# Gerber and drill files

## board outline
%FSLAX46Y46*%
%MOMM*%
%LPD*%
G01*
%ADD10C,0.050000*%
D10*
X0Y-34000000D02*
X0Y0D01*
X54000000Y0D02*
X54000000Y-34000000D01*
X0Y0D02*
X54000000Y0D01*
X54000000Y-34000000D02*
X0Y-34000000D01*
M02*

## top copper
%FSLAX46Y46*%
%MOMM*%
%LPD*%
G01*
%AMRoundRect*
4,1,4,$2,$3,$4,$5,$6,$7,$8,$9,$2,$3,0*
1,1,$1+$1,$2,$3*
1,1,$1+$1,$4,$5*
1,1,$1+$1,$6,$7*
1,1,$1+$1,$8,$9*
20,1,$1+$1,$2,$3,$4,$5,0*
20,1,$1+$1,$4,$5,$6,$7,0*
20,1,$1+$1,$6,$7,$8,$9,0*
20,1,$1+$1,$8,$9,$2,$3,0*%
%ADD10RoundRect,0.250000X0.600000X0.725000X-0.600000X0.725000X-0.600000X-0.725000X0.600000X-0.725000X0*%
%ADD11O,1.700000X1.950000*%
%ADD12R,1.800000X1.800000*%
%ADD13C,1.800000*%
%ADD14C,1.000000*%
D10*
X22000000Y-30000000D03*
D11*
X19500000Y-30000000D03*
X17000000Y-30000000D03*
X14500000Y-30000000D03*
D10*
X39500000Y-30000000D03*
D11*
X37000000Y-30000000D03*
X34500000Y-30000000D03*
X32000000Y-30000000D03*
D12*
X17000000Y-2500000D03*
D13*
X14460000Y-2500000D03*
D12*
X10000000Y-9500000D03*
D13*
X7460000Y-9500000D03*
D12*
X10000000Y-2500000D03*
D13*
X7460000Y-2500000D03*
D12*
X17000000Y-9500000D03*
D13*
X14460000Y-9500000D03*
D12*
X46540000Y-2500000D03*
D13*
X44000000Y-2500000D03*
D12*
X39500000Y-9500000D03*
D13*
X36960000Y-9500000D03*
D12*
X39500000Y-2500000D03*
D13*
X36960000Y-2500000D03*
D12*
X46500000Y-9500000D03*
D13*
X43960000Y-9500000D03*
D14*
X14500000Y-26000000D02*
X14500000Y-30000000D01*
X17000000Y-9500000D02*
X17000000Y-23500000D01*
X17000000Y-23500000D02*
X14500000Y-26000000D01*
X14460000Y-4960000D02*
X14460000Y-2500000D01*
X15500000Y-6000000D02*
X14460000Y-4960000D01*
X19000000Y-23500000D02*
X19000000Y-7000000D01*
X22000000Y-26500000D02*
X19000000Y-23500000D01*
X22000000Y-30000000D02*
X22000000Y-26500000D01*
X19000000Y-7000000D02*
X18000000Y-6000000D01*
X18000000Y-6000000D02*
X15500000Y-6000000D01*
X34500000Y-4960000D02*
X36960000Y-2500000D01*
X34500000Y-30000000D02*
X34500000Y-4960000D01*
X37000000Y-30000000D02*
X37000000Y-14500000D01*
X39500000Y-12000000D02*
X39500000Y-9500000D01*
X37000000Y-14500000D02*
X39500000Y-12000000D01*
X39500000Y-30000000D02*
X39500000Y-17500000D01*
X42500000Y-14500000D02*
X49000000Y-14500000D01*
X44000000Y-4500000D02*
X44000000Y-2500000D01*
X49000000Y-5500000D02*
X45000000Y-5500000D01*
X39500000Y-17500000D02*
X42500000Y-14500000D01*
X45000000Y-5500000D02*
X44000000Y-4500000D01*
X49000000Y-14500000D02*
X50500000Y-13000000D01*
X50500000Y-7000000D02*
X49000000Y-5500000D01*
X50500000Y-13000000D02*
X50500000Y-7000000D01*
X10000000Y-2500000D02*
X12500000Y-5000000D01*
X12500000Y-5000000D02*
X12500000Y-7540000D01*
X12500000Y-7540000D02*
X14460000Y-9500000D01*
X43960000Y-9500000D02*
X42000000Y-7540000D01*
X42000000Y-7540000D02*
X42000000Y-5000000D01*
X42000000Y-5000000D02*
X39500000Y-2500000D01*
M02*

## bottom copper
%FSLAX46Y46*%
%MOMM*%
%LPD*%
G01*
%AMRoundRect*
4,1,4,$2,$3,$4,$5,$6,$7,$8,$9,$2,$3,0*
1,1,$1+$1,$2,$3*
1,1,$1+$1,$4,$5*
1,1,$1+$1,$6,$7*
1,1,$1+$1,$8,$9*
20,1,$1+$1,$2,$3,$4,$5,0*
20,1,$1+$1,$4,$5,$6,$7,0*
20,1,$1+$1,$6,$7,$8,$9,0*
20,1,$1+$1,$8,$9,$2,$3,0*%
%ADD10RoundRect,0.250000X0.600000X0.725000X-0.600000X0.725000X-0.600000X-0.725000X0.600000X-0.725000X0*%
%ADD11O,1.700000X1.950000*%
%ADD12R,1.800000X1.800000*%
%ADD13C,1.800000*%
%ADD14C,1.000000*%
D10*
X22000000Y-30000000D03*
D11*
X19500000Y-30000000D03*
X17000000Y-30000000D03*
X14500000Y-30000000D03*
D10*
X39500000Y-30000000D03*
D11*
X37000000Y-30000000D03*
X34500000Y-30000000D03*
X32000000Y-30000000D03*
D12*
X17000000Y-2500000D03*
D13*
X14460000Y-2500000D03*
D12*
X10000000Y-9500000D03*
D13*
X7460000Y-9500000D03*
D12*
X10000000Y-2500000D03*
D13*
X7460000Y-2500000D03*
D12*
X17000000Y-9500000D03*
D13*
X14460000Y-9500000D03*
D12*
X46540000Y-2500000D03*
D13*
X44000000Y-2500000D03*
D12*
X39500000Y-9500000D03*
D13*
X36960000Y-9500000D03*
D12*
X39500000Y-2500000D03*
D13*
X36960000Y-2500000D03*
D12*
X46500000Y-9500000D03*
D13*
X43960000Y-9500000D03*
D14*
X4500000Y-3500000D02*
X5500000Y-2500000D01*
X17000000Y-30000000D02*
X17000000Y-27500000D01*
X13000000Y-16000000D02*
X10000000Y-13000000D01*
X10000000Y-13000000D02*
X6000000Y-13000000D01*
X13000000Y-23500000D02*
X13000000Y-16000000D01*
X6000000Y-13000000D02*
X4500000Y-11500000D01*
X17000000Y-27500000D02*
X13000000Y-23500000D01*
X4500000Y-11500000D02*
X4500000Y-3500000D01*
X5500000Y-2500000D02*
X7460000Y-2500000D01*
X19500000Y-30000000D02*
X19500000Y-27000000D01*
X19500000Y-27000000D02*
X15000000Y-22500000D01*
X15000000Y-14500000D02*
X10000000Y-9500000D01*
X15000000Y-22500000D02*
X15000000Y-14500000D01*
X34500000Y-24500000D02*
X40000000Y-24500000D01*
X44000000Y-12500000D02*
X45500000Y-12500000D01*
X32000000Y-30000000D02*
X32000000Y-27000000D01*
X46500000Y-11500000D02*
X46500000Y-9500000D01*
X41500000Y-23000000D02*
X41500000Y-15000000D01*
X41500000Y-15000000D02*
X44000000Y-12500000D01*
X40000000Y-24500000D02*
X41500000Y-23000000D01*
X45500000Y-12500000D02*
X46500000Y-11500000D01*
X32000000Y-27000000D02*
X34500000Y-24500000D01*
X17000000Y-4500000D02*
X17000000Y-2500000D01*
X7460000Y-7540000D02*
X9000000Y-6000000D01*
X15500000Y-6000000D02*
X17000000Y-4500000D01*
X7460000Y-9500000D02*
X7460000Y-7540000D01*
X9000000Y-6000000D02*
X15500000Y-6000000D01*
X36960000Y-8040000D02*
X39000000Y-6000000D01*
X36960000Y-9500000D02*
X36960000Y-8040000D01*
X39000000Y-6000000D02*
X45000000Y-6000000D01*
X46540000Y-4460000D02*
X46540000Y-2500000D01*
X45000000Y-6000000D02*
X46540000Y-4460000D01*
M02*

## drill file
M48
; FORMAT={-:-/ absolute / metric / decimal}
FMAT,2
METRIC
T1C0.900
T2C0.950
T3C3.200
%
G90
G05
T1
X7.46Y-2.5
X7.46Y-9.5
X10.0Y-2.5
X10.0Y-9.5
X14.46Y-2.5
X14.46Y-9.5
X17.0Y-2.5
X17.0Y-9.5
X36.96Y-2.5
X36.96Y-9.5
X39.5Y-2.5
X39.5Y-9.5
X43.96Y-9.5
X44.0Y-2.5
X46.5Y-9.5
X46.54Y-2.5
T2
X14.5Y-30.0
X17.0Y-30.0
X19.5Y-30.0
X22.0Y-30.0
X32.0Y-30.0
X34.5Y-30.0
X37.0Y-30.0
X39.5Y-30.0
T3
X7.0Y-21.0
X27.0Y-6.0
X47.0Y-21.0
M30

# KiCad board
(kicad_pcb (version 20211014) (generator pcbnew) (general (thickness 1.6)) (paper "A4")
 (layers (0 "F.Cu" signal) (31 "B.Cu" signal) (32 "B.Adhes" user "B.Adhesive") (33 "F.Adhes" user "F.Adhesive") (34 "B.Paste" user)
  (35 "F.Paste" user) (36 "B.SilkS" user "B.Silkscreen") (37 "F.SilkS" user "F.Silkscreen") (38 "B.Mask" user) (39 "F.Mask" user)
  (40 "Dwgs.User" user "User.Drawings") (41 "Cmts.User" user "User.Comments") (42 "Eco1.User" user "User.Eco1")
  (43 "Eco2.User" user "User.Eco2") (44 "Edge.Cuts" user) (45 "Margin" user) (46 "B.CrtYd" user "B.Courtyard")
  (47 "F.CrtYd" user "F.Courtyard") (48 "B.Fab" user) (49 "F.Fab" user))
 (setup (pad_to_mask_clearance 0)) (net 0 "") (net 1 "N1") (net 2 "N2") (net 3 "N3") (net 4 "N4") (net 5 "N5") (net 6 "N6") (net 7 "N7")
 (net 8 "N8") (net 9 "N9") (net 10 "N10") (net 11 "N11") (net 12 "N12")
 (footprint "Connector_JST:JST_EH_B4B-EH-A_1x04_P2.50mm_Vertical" (layer "F.Cu") (at 22 30 180)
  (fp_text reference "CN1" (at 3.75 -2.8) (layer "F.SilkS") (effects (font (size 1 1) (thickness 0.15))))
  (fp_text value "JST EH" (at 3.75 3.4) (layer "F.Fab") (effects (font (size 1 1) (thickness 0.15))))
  (pad "1" thru_hole roundrect locked (at 0 0 180) (size 1.7 1.95) (drill 0.95) (layers *.Cu *.Mask) (roundrect_rratio 0.147059)
   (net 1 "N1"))
  (pad "2" thru_hole oval locked (at 2.5 0 180) (size 1.7 1.95) (drill 0.95) (layers *.Cu *.Mask) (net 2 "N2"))
  (pad "3" thru_hole oval locked (at 5 0 180) (size 1.7 1.95) (drill 0.95) (layers *.Cu *.Mask) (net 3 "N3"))
  (pad "4" thru_hole oval locked (at 7.5 0 180) (size 1.7 1.95) (drill 0.95) (layers *.Cu *.Mask) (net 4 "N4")))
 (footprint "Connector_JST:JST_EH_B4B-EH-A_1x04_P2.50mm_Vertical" (layer "F.Cu") (at 39.5 30 180)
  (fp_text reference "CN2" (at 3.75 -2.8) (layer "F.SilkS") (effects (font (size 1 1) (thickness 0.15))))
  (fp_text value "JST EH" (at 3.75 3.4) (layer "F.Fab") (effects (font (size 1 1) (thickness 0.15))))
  (pad "1" thru_hole roundrect locked (at 0 0 180) (size 1.7 1.95) (drill 0.95) (layers *.Cu *.Mask) (roundrect_rratio 0.147059)
   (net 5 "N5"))
  (pad "2" thru_hole oval locked (at 2.5 0 180) (size 1.7 1.95) (drill 0.95) (layers *.Cu *.Mask) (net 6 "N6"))
  (pad "3" thru_hole oval locked (at 5 0 180) (size 1.7 1.95) (drill 0.95) (layers *.Cu *.Mask) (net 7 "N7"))
  (pad "4" thru_hole oval locked (at 7.5 0 180) (size 1.7 1.95) (drill 0.95) (layers *.Cu *.Mask) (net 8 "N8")))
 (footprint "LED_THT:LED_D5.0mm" (layer "F.Cu") (at 17 2.5 180)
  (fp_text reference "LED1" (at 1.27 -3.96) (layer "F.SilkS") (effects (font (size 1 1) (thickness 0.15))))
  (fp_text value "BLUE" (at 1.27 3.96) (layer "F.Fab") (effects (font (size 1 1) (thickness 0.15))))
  (pad "1" thru_hole rect locked (at 0 0 180) (size 1.8 1.8) (drill 0.9) (layers *.Cu *.Mask) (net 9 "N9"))
  (pad "2" thru_hole circle locked (at 2.54 0 180) (size 1.8 1.8) (drill 0.9) (layers *.Cu *.Mask) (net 1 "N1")))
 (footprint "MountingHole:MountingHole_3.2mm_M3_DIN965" (layer "F.Cu") (at 7 21)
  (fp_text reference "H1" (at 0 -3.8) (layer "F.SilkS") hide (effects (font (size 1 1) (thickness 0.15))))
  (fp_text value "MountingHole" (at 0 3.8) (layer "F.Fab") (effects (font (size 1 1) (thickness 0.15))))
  (pad "" np_thru_hole circle locked (at 0 0) (size 3.2 3.2) (drill 3.2) (layers *.Cu *.Mask)))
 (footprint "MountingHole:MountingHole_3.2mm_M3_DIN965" (layer "F.Cu") (at 27 6)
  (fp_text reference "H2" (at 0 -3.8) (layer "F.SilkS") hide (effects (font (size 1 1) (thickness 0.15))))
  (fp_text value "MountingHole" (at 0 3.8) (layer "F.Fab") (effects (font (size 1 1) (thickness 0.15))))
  (pad "" np_thru_hole circle locked (at 0 0) (size 3.2 3.2) (drill 3.2) (layers *.Cu *.Mask)))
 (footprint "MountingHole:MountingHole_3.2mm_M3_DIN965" (layer "F.Cu") (at 47 21)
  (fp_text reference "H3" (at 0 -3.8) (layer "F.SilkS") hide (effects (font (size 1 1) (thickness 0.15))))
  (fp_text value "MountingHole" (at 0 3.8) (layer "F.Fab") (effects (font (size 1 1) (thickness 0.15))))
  (pad "" np_thru_hole circle locked (at 0 0) (size 3.2 3.2) (drill 3.2) (layers *.Cu *.Mask)))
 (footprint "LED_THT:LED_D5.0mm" (layer "F.Cu") (at 10 9.5 180)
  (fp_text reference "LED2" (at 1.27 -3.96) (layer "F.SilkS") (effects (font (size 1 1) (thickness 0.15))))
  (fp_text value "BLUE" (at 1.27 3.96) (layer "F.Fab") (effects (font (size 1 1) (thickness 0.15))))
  (pad "1" thru_hole rect locked (at 0 0 180) (size 1.8 1.8) (drill 0.9) (layers *.Cu *.Mask) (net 2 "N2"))
  (pad "2" thru_hole circle locked (at 2.54 0 180) (size 1.8 1.8) (drill 0.9) (layers *.Cu *.Mask) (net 9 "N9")))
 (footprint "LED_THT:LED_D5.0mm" (layer "F.Cu") (at 10 2.5 180)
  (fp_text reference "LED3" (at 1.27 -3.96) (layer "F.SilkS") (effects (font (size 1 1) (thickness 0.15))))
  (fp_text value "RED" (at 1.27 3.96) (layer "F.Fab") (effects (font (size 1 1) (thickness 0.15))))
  (pad "1" thru_hole rect locked (at 0 0 180) (size 1.8 1.8) (drill 0.9) (layers *.Cu *.Mask) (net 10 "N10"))
  (pad "2" thru_hole circle locked (at 2.54 0 180) (size 1.8 1.8) (drill 0.9) (layers *.Cu *.Mask) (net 3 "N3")))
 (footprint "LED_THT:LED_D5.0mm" (layer "F.Cu") (at 17 9.5 180)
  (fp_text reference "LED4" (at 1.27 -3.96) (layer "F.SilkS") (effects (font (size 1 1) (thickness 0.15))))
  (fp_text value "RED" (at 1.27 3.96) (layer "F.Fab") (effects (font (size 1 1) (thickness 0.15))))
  (pad "1" thru_hole rect locked (at 0 0 180) (size 1.8 1.8) (drill 0.9) (layers *.Cu *.Mask) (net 4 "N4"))
  (pad "2" thru_hole circle locked (at 2.54 0 180) (size 1.8 1.8) (drill 0.9) (layers *.Cu *.Mask) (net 10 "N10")))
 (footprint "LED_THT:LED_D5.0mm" (layer "F.Cu") (at 46.54 2.5 180)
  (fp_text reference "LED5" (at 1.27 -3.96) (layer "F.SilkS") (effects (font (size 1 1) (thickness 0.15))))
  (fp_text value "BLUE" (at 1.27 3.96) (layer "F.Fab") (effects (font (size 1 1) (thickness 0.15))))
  (pad "1" thru_hole rect locked (at 0 0 180) (size 1.8 1.8) (drill 0.9) (layers *.Cu *.Mask) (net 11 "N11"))
  (pad "2" thru_hole circle locked (at 2.54 0 180) (size 1.8 1.8) (drill 0.9) (layers *.Cu *.Mask) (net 5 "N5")))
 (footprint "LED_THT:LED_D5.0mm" (layer "F.Cu") (at 39.5 9.5 180)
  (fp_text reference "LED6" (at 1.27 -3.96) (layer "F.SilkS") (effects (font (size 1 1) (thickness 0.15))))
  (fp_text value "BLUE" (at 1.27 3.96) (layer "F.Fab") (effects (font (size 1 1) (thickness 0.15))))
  (pad "1" thru_hole rect locked (at 0 0 180) (size 1.8 1.8) (drill 0.9) (layers *.Cu *.Mask) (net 6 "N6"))
  (pad "2" thru_hole circle locked (at 2.54 0 180) (size 1.8 1.8) (drill 0.9) (layers *.Cu *.Mask) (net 11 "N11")))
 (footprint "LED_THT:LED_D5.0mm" (layer "F.Cu") (at 39.5 2.5 180)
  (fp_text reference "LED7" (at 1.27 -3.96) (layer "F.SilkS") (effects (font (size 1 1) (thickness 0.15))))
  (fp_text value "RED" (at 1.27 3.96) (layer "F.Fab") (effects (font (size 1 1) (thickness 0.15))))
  (pad "1" thru_hole rect locked (at 0 0 180) (size 1.8 1.8) (drill 0.9) (layers *.Cu *.Mask) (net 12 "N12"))
  (pad "2" thru_hole circle locked (at 2.54 0 180) (size 1.8 1.8) (drill 0.9) (layers *.Cu *.Mask) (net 7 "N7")))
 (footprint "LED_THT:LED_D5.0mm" (layer "F.Cu") (at 46.5 9.5 180)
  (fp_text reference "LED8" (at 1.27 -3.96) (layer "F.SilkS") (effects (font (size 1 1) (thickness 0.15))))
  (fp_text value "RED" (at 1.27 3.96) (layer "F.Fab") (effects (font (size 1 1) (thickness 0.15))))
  (pad "1" thru_hole rect locked (at 0 0 180) (size 1.8 1.8) (drill 0.9) (layers *.Cu *.Mask) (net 8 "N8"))
  (pad "2" thru_hole circle locked (at 2.54 0 180) (size 1.8 1.8) (drill 0.9) (layers *.Cu *.Mask) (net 12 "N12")))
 (gr_line (start 0 34) (end 0 0) (layer "Edge.Cuts") (width 0.05))
 (gr_line (start 54 0) (end 54 34) (layer "Edge.Cuts") (width 0.05))
 (gr_line (start 0 0) (end 54 0) (layer "Edge.Cuts") (width 0.05))
 (gr_line (start 54 34) (end 0 34) (layer "Edge.Cuts") (width 0.05))
 (segment (start 14.5 26) (end 14.5 30) (width 1) (layer "F.Cu") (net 4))
 (segment (start 17 9.5) (end 17 23.5) (width 1) (layer "F.Cu") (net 4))
 (segment (start 17 23.5) (end 14.5 26) (width 1) (layer "F.Cu") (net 4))
 (segment (start 4.5 3.5) (end 5.5 2.5) (width 1) (layer "B.Cu") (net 3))
 (segment (start 17 30) (end 17 27.5) (width 1) (layer "B.Cu") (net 3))
 (segment (start 13 16) (end 10 13) (width 1) (layer "B.Cu") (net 3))
 (segment (start 10 13) (end 6 13) (width 1) (layer "B.Cu") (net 3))
 (segment (start 13 23.5) (end 13 16) (width 1) (layer "B.Cu") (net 3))
 (segment (start 6 13) (end 4.5 11.5) (width 1) (layer "B.Cu") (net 3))
 (segment (start 17 27.5) (end 13 23.5) (width 1) (layer "B.Cu") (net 3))
 (segment (start 4.5 11.5) (end 4.5 3.5) (width 1) (layer "B.Cu") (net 3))
 (segment (start 5.5 2.5) (end 7.46 2.5) (width 1) (layer "B.Cu") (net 3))
 (segment (start 19.5 30) (end 19.5 27) (width 1) (layer "B.Cu") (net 2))
 (segment (start 19.5 27) (end 15 22.5) (width 1) (layer "B.Cu") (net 2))
 (segment (start 15 14.5) (end 10 9.5) (width 1) (layer "B.Cu") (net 2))
 (segment (start 15 22.5) (end 15 14.5) (width 1) (layer "B.Cu") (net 2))
 (segment (start 14.46 4.96) (end 14.46 2.5) (width 1) (layer "F.Cu") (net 1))
 (segment (start 15.5 6) (end 14.46 4.96) (width 1) (layer "F.Cu") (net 1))
 (segment (start 19 23.5) (end 19 7) (width 1) (layer "F.Cu") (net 1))
 (segment (start 22 26.5) (end 19 23.5) (width 1) (layer "F.Cu") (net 1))
 (segment (start 22 30) (end 22 26.5) (width 1) (layer "F.Cu") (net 1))
 (segment (start 19 7) (end 18 6) (width 1) (layer "F.Cu") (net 1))
 (segment (start 18 6) (end 15.5 6) (width 1) (layer "F.Cu") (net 1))
 (segment (start 34.5 24.5) (end 40 24.5) (width 1) (layer "B.Cu") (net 8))
 (segment (start 44 12.5) (end 45.5 12.5) (width 1) (layer "B.Cu") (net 8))
 (segment (start 32 30) (end 32 27) (width 1) (layer "B.Cu") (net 8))
 (segment (start 46.5 11.5) (end 46.5 9.5) (width 1) (layer "B.Cu") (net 8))
 (segment (start 41.5 23) (end 41.5 15) (width 1) (layer "B.Cu") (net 8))
 (segment (start 41.5 15) (end 44 12.5) (width 1) (layer "B.Cu") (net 8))
 (segment (start 40 24.5) (end 41.5 23) (width 1) (layer "B.Cu") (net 8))
 (segment (start 45.5 12.5) (end 46.5 11.5) (width 1) (layer "B.Cu") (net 8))
 (segment (start 32 27) (end 34.5 24.5) (width 1) (layer "B.Cu") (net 8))
 (segment (start 34.5 4.96) (end 36.96 2.5) (width 1) (layer "F.Cu") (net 7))
 (segment (start 34.5 30) (end 34.5 4.96) (width 1) (layer "F.Cu") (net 7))
 (segment (start 37 30) (end 37 14.5) (width 1) (layer "F.Cu") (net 6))
 (segment (start 39.5 12) (end 39.5 9.5) (width 1) (layer "F.Cu") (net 6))
 (segment (start 37 14.5) (end 39.5 12) (width 1) (layer "F.Cu") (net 6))
 (segment (start 39.5 30) (end 39.5 17.5) (width 1) (layer "F.Cu") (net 5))
 (segment (start 42.5 14.5) (end 49 14.5) (width 1) (layer "F.Cu") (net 5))
 (segment (start 44 4.5) (end 44 2.5) (width 1) (layer "F.Cu") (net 5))
 (segment (start 49 5.5) (end 45 5.5) (width 1) (layer "F.Cu") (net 5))
 (segment (start 39.5 17.5) (end 42.5 14.5) (width 1) (layer "F.Cu") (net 5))
 (segment (start 45 5.5) (end 44 4.5) (width 1) (layer "F.Cu") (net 5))
 (segment (start 49 14.5) (end 50.5 13) (width 1) (layer "F.Cu") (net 5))
 (segment (start 50.5 7) (end 49 5.5) (width 1) (layer "F.Cu") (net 5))
 (segment (start 50.5 13) (end 50.5 7) (width 1) (layer "F.Cu") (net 5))
 (segment (start 17 4.5) (end 17 2.5) (width 1) (layer "B.Cu") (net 9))
 (segment (start 7.46 7.54) (end 9 6) (width 1) (layer "B.Cu") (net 9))
 (segment (start 15.5 6) (end 17 4.5) (width 1) (layer "B.Cu") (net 9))
 (segment (start 7.46 9.5) (end 7.46 7.54) (width 1) (layer "B.Cu") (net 9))
 (segment (start 9 6) (end 15.5 6) (width 1) (layer "B.Cu") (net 9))
 (segment (start 10 2.5) (end 12.5 5) (width 1) (layer "F.Cu") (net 10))
 (segment (start 12.5 5) (end 12.5 7.54) (width 1) (layer "F.Cu") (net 10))
 (segment (start 12.5 7.54) (end 14.46 9.5) (width 1) (layer "F.Cu") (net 10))
 (segment (start 36.96 8.04) (end 39 6) (width 1) (layer "B.Cu") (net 11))
 (segment (start 36.96 9.5) (end 36.96 8.04) (width 1) (layer "B.Cu") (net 11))
 (segment (start 39 6) (end 45 6) (width 1) (layer "B.Cu") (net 11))
 (segment (start 46.54 4.46) (end 46.54 2.5) (width 1) (layer "B.Cu") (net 11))
 (segment (start 45 6) (end 46.54 4.46) (width 1) (layer "B.Cu") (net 11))
 (segment (start 43.96 9.5) (end 42 7.54) (width 1) (layer "F.Cu") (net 12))
 (segment (start 42 7.54) (end 42 5) (width 1) (layer "F.Cu") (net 12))
 (segment (start 42 5) (end 39.5 2.5) (width 1) (layer "F.Cu") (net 12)))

